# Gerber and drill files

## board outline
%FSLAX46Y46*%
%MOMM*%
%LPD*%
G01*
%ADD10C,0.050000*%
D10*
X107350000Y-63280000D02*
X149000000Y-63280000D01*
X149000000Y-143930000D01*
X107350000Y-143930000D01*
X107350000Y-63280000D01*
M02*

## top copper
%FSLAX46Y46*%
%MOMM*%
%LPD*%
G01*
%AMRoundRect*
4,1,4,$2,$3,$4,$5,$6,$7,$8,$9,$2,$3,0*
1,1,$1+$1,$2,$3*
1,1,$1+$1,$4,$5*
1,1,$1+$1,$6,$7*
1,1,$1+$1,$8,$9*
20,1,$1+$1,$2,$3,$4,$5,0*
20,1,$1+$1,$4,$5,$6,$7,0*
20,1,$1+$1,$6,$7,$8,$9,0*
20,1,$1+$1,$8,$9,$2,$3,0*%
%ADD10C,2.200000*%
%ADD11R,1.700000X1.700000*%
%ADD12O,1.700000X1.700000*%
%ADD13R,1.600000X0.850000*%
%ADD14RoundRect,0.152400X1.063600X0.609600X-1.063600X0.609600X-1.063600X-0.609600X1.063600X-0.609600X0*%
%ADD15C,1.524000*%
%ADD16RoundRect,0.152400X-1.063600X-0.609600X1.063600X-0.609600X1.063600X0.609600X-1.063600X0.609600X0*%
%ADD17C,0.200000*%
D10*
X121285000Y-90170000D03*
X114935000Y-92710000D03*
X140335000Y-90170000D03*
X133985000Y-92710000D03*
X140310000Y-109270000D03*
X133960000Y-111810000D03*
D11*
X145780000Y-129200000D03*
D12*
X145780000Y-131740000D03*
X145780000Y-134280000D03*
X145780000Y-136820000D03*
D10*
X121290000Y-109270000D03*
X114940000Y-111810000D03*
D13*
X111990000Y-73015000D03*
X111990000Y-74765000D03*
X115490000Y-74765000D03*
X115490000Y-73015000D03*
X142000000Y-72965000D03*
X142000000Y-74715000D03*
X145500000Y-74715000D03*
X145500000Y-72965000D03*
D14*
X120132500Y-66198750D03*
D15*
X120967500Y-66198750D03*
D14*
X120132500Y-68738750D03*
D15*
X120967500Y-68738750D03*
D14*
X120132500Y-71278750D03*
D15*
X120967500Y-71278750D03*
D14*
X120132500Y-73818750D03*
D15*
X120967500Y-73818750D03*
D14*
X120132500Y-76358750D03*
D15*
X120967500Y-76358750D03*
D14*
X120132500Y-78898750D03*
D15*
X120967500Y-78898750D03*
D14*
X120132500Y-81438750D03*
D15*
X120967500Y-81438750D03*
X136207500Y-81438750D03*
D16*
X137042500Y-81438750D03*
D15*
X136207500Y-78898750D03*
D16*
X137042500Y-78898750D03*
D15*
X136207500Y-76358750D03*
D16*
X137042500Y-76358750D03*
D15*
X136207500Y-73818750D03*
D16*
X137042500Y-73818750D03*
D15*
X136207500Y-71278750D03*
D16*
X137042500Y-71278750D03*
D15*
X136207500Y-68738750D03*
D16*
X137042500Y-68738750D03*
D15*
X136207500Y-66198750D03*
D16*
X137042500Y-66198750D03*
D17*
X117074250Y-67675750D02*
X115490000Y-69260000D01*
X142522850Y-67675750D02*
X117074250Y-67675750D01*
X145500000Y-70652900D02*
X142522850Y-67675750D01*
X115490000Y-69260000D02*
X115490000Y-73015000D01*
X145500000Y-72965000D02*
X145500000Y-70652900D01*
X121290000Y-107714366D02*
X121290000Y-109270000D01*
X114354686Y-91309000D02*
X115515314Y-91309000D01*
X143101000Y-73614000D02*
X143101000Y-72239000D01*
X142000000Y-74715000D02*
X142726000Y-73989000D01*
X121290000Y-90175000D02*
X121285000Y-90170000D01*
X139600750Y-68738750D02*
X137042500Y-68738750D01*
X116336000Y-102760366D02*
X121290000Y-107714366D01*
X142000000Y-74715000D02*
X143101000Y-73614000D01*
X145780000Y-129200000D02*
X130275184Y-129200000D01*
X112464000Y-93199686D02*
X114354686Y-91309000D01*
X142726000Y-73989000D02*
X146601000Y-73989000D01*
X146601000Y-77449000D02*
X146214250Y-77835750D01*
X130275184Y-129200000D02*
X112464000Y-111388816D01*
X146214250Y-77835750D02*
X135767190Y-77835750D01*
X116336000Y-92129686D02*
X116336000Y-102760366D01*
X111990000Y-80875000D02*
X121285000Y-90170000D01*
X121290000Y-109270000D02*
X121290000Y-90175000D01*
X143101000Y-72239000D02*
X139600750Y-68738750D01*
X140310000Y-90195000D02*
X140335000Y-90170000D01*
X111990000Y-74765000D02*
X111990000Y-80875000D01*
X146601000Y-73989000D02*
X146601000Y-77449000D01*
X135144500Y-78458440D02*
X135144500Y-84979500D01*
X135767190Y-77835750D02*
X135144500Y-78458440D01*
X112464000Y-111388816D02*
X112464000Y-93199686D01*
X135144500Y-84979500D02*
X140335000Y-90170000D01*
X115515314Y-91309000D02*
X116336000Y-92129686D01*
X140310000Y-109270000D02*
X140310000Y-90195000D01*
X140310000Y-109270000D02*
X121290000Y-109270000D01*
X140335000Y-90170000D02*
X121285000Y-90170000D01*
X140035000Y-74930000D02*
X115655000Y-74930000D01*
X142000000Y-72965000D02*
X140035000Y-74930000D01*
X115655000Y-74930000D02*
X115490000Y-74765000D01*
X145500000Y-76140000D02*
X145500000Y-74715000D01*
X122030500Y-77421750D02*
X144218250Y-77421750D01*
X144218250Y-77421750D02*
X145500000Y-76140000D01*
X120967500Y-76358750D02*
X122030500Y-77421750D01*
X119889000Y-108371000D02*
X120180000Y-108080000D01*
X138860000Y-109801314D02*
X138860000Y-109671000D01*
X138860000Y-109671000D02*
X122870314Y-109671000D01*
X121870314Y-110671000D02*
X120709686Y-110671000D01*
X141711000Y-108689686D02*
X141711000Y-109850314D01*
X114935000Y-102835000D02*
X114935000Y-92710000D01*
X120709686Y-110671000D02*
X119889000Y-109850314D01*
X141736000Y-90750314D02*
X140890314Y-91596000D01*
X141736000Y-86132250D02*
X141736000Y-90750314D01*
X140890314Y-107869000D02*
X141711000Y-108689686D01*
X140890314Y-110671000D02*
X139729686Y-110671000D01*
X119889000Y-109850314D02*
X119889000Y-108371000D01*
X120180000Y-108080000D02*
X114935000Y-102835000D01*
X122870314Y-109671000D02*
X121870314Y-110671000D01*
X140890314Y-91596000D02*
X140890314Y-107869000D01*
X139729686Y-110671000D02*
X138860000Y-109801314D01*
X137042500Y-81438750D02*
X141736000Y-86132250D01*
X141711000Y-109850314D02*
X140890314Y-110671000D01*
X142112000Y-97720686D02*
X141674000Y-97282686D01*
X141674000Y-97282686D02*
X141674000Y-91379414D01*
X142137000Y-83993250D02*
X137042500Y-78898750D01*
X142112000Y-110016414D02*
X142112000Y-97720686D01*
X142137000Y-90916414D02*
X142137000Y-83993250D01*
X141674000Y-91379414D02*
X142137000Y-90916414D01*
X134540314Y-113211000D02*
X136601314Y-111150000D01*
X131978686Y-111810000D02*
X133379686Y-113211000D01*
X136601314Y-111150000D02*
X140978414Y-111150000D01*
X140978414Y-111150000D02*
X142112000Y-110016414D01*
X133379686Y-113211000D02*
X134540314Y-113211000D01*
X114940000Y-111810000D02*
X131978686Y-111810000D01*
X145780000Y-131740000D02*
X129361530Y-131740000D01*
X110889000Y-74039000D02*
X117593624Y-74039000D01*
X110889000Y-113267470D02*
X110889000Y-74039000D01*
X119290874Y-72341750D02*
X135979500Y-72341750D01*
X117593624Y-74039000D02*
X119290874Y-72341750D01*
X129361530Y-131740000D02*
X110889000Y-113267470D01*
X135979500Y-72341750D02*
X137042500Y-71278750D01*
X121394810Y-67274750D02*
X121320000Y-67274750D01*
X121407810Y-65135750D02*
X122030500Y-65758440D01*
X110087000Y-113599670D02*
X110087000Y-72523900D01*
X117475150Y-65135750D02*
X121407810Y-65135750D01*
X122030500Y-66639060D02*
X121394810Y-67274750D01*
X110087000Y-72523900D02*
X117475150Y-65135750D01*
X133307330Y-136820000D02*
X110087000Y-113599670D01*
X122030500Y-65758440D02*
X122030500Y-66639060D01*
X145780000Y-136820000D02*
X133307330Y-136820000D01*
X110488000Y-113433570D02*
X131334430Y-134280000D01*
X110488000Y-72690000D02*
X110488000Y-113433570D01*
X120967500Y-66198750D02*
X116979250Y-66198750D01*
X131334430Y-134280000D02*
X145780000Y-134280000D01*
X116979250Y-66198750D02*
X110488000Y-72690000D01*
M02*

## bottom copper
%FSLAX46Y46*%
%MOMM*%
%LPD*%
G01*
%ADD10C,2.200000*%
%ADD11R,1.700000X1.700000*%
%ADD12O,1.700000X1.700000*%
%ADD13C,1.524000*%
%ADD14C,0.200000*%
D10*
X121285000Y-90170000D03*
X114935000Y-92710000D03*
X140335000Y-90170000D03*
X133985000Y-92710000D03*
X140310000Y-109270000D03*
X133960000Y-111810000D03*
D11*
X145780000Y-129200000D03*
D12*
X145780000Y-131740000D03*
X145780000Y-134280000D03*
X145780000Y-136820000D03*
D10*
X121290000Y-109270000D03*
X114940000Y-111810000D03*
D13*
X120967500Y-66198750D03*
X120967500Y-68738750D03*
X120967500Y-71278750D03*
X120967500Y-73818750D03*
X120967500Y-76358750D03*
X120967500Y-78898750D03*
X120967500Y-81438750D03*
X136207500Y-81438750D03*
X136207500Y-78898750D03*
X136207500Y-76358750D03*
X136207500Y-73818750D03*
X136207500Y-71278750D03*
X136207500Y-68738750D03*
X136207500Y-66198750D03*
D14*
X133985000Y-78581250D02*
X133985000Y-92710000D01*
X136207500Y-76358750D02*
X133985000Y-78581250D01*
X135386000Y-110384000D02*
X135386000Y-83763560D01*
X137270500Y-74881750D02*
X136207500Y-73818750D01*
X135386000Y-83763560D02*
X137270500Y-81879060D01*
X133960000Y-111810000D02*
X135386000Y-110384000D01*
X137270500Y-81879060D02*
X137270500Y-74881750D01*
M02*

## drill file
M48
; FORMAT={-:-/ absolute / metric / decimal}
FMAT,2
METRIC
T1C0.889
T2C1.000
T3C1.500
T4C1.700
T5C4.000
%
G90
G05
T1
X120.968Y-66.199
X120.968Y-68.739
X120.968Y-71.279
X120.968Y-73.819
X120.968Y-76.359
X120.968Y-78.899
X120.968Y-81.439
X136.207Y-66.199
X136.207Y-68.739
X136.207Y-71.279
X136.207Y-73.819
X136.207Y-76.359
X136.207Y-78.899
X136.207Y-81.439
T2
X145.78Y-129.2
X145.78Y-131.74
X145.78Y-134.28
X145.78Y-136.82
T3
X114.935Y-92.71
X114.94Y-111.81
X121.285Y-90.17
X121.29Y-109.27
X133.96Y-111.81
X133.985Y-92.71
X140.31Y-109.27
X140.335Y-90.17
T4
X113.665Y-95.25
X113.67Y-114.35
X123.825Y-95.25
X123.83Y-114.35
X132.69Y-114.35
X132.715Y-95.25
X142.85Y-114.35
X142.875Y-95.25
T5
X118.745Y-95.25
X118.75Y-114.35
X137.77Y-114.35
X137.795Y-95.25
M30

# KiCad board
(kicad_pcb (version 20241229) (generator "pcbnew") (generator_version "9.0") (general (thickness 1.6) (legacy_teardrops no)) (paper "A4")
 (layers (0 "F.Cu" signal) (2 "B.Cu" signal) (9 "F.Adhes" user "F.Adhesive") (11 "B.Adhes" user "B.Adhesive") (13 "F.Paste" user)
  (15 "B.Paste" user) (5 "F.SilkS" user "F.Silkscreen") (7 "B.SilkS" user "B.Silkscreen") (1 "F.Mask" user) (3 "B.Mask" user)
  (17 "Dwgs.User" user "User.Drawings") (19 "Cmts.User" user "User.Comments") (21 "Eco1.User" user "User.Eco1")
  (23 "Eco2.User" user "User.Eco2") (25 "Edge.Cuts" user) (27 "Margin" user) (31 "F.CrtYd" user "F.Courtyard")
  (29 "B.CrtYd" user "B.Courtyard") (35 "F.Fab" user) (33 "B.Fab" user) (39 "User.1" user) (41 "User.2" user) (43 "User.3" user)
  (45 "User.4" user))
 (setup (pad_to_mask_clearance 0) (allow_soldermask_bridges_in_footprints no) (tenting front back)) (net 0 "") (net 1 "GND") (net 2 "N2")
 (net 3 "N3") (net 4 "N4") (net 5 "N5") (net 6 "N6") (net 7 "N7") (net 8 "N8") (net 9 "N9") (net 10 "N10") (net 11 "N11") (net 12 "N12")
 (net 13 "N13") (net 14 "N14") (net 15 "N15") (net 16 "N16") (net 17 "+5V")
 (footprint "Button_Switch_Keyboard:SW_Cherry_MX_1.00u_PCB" (layer "F.Cu") (at 121.285 90.17)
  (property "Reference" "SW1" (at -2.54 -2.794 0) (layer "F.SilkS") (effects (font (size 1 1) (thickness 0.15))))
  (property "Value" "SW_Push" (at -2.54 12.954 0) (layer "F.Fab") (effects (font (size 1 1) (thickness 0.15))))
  (pad "" np_thru_hole circle (at -7.62 5.08) (size 1.7 1.7) (drill 1.7) (layers "*.Cu" "*.Mask"))
  (pad "" np_thru_hole circle (at -2.54 5.08) (size 4 4) (drill 4) (layers "*.Cu" "*.Mask"))
  (pad "" np_thru_hole circle (at 2.54 5.08) (size 1.7 1.7) (drill 1.7) (layers "*.Cu" "*.Mask"))
  (pad "1" thru_hole circle (at 0 0) (size 2.2 2.2) (drill 1.5) (layers "*.Cu" "*.Mask") (remove_unused_layers no) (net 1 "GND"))
  (pad "2" thru_hole circle (at -6.35 2.54) (size 2.2 2.2) (drill 1.5) (layers "*.Cu" "*.Mask") (remove_unused_layers no) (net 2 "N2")))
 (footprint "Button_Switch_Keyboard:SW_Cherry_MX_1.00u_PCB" (layer "F.Cu") (at 140.335 90.17)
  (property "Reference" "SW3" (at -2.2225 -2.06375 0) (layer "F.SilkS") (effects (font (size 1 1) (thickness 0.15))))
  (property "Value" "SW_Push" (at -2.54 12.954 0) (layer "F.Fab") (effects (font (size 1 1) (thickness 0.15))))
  (pad "" np_thru_hole circle (at -7.62 5.08) (size 1.7 1.7) (drill 1.7) (layers "*.Cu" "*.Mask"))
  (pad "" np_thru_hole circle (at -2.54 5.08) (size 4 4) (drill 4) (layers "*.Cu" "*.Mask"))
  (pad "" np_thru_hole circle (at 2.54 5.08) (size 1.7 1.7) (drill 1.7) (layers "*.Cu" "*.Mask"))
  (pad "1" thru_hole circle (at 0 0) (size 2.2 2.2) (drill 1.5) (layers "*.Cu" "*.Mask") (remove_unused_layers no) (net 1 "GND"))
  (pad "2" thru_hole circle (at -6.35 2.54) (size 2.2 2.2) (drill 1.5) (layers "*.Cu" "*.Mask") (remove_unused_layers no) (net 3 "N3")))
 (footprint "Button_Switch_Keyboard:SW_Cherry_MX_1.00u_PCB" (layer "F.Cu") (at 140.31 109.27)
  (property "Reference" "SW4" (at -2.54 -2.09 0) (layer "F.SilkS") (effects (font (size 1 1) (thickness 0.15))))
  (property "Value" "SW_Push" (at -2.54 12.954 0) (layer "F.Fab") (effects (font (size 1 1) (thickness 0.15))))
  (pad "" np_thru_hole circle (at -7.62 5.08) (size 1.7 1.7) (drill 1.7) (layers "*.Cu" "*.Mask"))
  (pad "" np_thru_hole circle (at -2.54 5.08) (size 4 4) (drill 4) (layers "*.Cu" "*.Mask"))
  (pad "" np_thru_hole circle (at 2.54 5.08) (size 1.7 1.7) (drill 1.7) (layers "*.Cu" "*.Mask"))
  (pad "1" thru_hole circle (at 0 0) (size 2.2 2.2) (drill 1.5) (layers "*.Cu" "*.Mask") (remove_unused_layers no) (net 1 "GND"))
  (pad "2" thru_hole circle (at -6.35 2.54) (size 2.2 2.2) (drill 1.5) (layers "*.Cu" "*.Mask") (remove_unused_layers no) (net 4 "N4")))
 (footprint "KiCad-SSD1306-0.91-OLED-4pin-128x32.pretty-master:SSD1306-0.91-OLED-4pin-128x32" (layer "F.Cu") (at 109.28 127.01)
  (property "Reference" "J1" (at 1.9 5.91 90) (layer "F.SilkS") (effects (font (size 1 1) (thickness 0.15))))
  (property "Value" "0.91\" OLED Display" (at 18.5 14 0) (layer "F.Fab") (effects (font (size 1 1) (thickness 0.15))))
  (pad "1" thru_hole rect (at 36.5 2.19) (size 1.7 1.7) (drill 1) (layers "*.Cu" "*.Mask") (remove_unused_layers no) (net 1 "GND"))
  (pad "2" thru_hole oval (at 36.5 4.73) (size 1.7 1.7) (drill 1) (layers "*.Cu" "*.Mask") (remove_unused_layers no) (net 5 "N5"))
  (pad "3" thru_hole oval (at 36.5 7.27) (size 1.7 1.7) (drill 1) (layers "*.Cu" "*.Mask") (remove_unused_layers no) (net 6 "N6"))
  (pad "4" thru_hole oval (at 36.5 9.81) (size 1.7 1.7) (drill 1) (layers "*.Cu" "*.Mask") (remove_unused_layers no) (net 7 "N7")))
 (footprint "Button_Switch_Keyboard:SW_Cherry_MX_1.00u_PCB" (layer "F.Cu") (at 121.29 109.27)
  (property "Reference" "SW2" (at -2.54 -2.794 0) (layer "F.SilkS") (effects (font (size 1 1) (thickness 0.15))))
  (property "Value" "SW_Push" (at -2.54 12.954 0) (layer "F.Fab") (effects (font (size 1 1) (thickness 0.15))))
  (pad "" np_thru_hole circle (at -7.62 5.08) (size 1.7 1.7) (drill 1.7) (layers "*.Cu" "*.Mask"))
  (pad "" np_thru_hole circle (at -2.54 5.08) (size 4 4) (drill 4) (layers "*.Cu" "*.Mask"))
  (pad "" np_thru_hole circle (at 2.54 5.08) (size 1.7 1.7) (drill 1.7) (layers "*.Cu" "*.Mask"))
  (pad "1" thru_hole circle (at 0 0) (size 2.2 2.2) (drill 1.5) (layers "*.Cu" "*.Mask") (remove_unused_layers no) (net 1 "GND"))
  (pad "2" thru_hole circle (at -6.35 2.54) (size 2.2 2.2) (drill 1.5) (layers "*.Cu" "*.Mask") (remove_unused_layers no) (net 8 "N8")))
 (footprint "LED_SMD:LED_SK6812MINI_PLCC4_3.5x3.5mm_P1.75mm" (layer "F.Cu") (at 113.74 73.89)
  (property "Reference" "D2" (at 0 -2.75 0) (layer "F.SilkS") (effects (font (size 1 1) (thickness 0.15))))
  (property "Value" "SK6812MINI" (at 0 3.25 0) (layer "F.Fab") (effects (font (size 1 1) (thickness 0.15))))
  (pad "1" smd rect (at -1.75 -0.875) (size 1.6 0.85) (layers "F.Cu" "F.Mask" "F.Paste") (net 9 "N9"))
  (pad "2" smd rect (at -1.75 0.875) (size 1.6 0.85) (layers "F.Cu" "F.Mask" "F.Paste") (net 1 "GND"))
  (pad "3" smd rect (at 1.75 0.875) (size 1.6 0.85) (layers "F.Cu" "F.Mask" "F.Paste") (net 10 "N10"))
  (pad "4" smd rect (at 1.75 -0.875) (size 1.6 0.85) (layers "F.Cu" "F.Mask" "F.Paste") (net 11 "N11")))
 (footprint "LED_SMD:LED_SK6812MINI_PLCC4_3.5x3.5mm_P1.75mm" (layer "F.Cu") (at 143.75 73.84)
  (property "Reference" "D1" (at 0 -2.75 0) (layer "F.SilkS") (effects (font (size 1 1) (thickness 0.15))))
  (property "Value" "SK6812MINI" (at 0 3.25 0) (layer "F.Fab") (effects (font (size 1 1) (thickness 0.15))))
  (pad "1" smd rect (at -1.75 -0.875) (size 1.6 0.85) (layers "F.Cu" "F.Mask" "F.Paste") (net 10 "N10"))
  (pad "2" smd rect (at -1.75 0.875) (size 1.6 0.85) (layers "F.Cu" "F.Mask" "F.Paste") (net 1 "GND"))
  (pad "3" smd rect (at 1.75 0.875) (size 1.6 0.85) (layers "F.Cu" "F.Mask" "F.Paste") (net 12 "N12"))
  (pad "4" smd rect (at 1.75 -0.875) (size 1.6 0.85) (layers "F.Cu" "F.Mask" "F.Paste") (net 11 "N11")))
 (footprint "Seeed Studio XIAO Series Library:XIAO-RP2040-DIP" (layer "F.Cu") (at 128.5875 73.81875)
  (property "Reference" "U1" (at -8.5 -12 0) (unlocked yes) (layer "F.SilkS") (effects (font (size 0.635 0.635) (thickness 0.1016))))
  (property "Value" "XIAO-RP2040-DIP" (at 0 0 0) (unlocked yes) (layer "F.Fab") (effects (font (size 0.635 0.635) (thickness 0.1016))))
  (pad "1" smd roundrect (at -8.455 -7.62 180) (size 2.432 1.524) (layers "F.Cu" "F.Mask") (roundrect_rratio 0.1) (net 6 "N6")
   (thermal_bridge_angle 45))
  (pad "1" thru_hole circle (at -7.62 -7.62 180) (size 1.524 1.524) (drill 0.889) (layers "*.Cu" "*.Mask") (remove_unused_layers no)
   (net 6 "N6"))
  (pad "2" smd roundrect (at -8.455 -5.08 180) (size 2.432 1.524) (layers "F.Cu" "F.Mask") (roundrect_rratio 0.1) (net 7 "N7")
   (thermal_bridge_angle 45))
  (pad "2" thru_hole circle (at -7.62 -5.08 180) (size 1.524 1.524) (drill 0.889) (layers "*.Cu" "*.Mask") (remove_unused_layers no)
   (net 7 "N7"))
  (pad "3" smd roundrect (at -8.455 -2.54 180) (size 2.432 1.524) (layers "F.Cu" "F.Mask") (roundrect_rratio 0.1) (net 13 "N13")
   (thermal_bridge_angle 45))
  (pad "3" thru_hole circle (at -7.62 -2.54 180) (size 1.524 1.524) (drill 0.889) (layers "*.Cu" "*.Mask") (remove_unused_layers no)
   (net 13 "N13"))
  (pad "4" smd roundrect (at -8.455 0 180) (size 2.432 1.524) (layers "F.Cu" "F.Mask") (roundrect_rratio 0.1) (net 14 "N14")
   (thermal_bridge_angle 45))
  (pad "4" thru_hole circle (at -7.62 0 180) (size 1.524 1.524) (drill 0.889) (layers "*.Cu" "*.Mask") (remove_unused_layers no)
   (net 14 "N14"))
  (pad "5" smd roundrect (at -8.455 2.54 180) (size 2.432 1.524) (layers "F.Cu" "F.Mask") (roundrect_rratio 0.1) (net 12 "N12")
   (thermal_bridge_angle 45))
  (pad "5" thru_hole circle (at -7.62 2.54 180) (size 1.524 1.524) (drill 0.889) (layers "*.Cu" "*.Mask") (remove_unused_layers no)
   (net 12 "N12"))
  (pad "6" smd roundrect (at -8.455 5.08 180) (size 2.432 1.524) (layers "F.Cu" "F.Mask") (roundrect_rratio 0.1) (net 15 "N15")
   (thermal_bridge_angle 45))
  (pad "6" thru_hole circle (at -7.62 5.08 180) (size 1.524 1.524) (drill 0.889) (layers "*.Cu" "*.Mask") (remove_unused_layers no)
   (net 15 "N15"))
  (pad "7" smd roundrect (at -8.455 7.62 180) (size 2.432 1.524) (layers "F.Cu" "F.Mask") (roundrect_rratio 0.1) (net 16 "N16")
   (thermal_bridge_angle 45))
  (pad "7" thru_hole circle (at -7.62 7.62 180) (size 1.524 1.524) (drill 0.889) (layers "*.Cu" "*.Mask") (remove_unused_layers no)
   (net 16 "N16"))
  (pad "8" thru_hole circle (at 7.62 7.62) (size 1.524 1.524) (drill 0.889) (layers "*.Cu" "*.Mask") (remove_unused_layers no) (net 2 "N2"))
  (pad "8" smd roundrect (at 8.455 7.62) (size 2.432 1.524) (layers "F.Cu" "F.Mask") (roundrect_rratio 0.1) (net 2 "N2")
   (thermal_bridge_angle 45))
  (pad "9" thru_hole circle (at 7.62 5.08) (size 1.524 1.524) (drill 0.889) (layers "*.Cu" "*.Mask") (remove_unused_layers no) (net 8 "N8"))
  (pad "9" smd roundrect (at 8.455 5.08) (size 2.432 1.524) (layers "F.Cu" "F.Mask") (roundrect_rratio 0.1) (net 8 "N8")
   (thermal_bridge_angle 45))
  (pad "10" thru_hole circle (at 7.62 2.54) (size 1.524 1.524) (drill 0.889) (layers "*.Cu" "*.Mask") (remove_unused_layers no) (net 3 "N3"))
  (pad "10" smd roundrect (at 8.455 2.54) (size 2.432 1.524) (layers "F.Cu" "F.Mask") (roundrect_rratio 0.1) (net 3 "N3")
   (thermal_bridge_angle 45))
  (pad "11" thru_hole circle (at 7.62 0) (size 1.524 1.524) (drill 0.889) (layers "*.Cu" "*.Mask") (remove_unused_layers no) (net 4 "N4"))
  (pad "11" smd roundrect (at 8.455 0) (size 2.432 1.524) (layers "F.Cu" "F.Mask") (roundrect_rratio 0.1) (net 4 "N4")
   (thermal_bridge_angle 45))
  (pad "12" thru_hole circle (at 7.62 -2.54) (size 1.524 1.524) (drill 0.889) (layers "*.Cu" "*.Mask") (remove_unused_layers no)
   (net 5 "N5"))
  (pad "12" smd roundrect (at 8.455 -2.54) (size 2.432 1.524) (layers "F.Cu" "F.Mask") (roundrect_rratio 0.1) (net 5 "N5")
   (thermal_bridge_angle 45))
  (pad "13" thru_hole circle (at 7.62 -5.08) (size 1.524 1.524) (drill 0.889) (layers "*.Cu" "*.Mask") (remove_unused_layers no)
   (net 1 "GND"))
  (pad "13" smd roundrect (at 8.455 -5.08) (size 2.432 1.524) (layers "F.Cu" "F.Mask") (roundrect_rratio 0.1) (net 1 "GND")
   (thermal_bridge_angle 45))
  (pad "14" thru_hole circle (at 7.62 -7.62) (size 1.524 1.524) (drill 0.889) (layers "*.Cu" "*.Mask") (remove_unused_layers no)
   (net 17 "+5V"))
  (pad "14" smd roundrect (at 8.455 -7.62) (size 2.432 1.524) (layers "F.Cu" "F.Mask") (roundrect_rratio 0.1) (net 17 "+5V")
   (thermal_bridge_angle 45)))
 (gr_rect (start 107.35 63.28) (end 149 143.93) (stroke (width 0.05) (type default)) (fill no) (layer "Edge.Cuts"))
 (segment (start 117.07425 67.67575) (end 115.49 69.26) (width 0.2) (layer "F.Cu") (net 11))
 (segment (start 142.52285 67.67575) (end 117.07425 67.67575) (width 0.2) (layer "F.Cu") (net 11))
 (segment (start 145.5 70.6529) (end 142.52285 67.67575) (width 0.2) (layer "F.Cu") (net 11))
 (segment (start 115.49 69.26) (end 115.49 73.015) (width 0.2) (layer "F.Cu") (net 11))
 (segment (start 145.5 72.965) (end 145.5 70.6529) (width 0.2) (layer "F.Cu") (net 11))
 (segment (start 121.29 107.714366) (end 121.29 109.27) (width 0.2) (layer "F.Cu") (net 1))
 (segment (start 114.354686 91.309) (end 115.515314 91.309) (width 0.2) (layer "F.Cu") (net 1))
 (segment (start 143.101 73.614) (end 143.101 72.239) (width 0.2) (layer "F.Cu") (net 1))
 (segment (start 142 74.715) (end 142.726 73.989) (width 0.2) (layer "F.Cu") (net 1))
 (segment (start 121.29 90.175) (end 121.285 90.17) (width 0.2) (layer "F.Cu") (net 1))
 (segment (start 139.60075 68.73875) (end 137.0425 68.73875) (width 0.2) (layer "F.Cu") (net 1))
 (segment (start 116.336 102.760366) (end 121.29 107.714366) (width 0.2) (layer "F.Cu") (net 1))
 (segment (start 142 74.715) (end 143.101 73.614) (width 0.2) (layer "F.Cu") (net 1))
 (segment (start 145.78 129.2) (end 130.275184 129.2) (width 0.2) (layer "F.Cu") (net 1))
 (segment (start 112.464 93.199686) (end 114.354686 91.309) (width 0.2) (layer "F.Cu") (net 1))
 (segment (start 142.726 73.989) (end 146.601 73.989) (width 0.2) (layer "F.Cu") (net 1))
 (segment (start 146.601 77.449) (end 146.21425 77.83575) (width 0.2) (layer "F.Cu") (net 1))
 (segment (start 130.275184 129.2) (end 112.464 111.388816) (width 0.2) (layer "F.Cu") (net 1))
 (segment (start 146.21425 77.83575) (end 135.76719 77.83575) (width 0.2) (layer "F.Cu") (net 1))
 (segment (start 116.336 92.129686) (end 116.336 102.760366) (width 0.2) (layer "F.Cu") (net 1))
 (segment (start 111.99 80.875) (end 121.285 90.17) (width 0.2) (layer "F.Cu") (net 1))
 (segment (start 121.29 109.27) (end 121.29 90.175) (width 0.2) (layer "F.Cu") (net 1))
 (segment (start 143.101 72.239) (end 139.60075 68.73875) (width 0.2) (layer "F.Cu") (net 1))
 (segment (start 140.31 90.195) (end 140.335 90.17) (width 0.2) (layer "F.Cu") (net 1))
 (segment (start 111.99 74.765) (end 111.99 80.875) (width 0.2) (layer "F.Cu") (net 1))
 (segment (start 146.601 73.989) (end 146.601 77.449) (width 0.2) (layer "F.Cu") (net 1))
 (segment (start 135.1445 78.45844) (end 135.1445 84.9795) (width 0.2) (layer "F.Cu") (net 1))
 (segment (start 135.76719 77.83575) (end 135.1445 78.45844) (width 0.2) (layer "F.Cu") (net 1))
 (segment (start 112.464 111.388816) (end 112.464 93.199686) (width 0.2) (layer "F.Cu") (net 1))
 (segment (start 135.1445 84.9795) (end 140.335 90.17) (width 0.2) (layer "F.Cu") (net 1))
 (segment (start 115.515314 91.309) (end 116.336 92.129686) (width 0.2) (layer "F.Cu") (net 1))
 (segment (start 140.31 109.27) (end 140.31 90.195) (width 0.2) (layer "F.Cu") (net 1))
 (segment (start 140.31 109.27) (end 121.29 109.27) (width 0.2) (layer "F.Cu") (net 1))
 (segment (start 140.335 90.17) (end 121.285 90.17) (width 0.2) (layer "F.Cu") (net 1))
 (segment (start 140.035 74.93) (end 115.655 74.93) (width 0.2) (layer "F.Cu") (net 10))
 (segment (start 142 72.965) (end 140.035 74.93) (width 0.2) (layer "F.Cu") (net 10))
 (segment (start 115.655 74.93) (end 115.49 74.765) (width 0.2) (layer "F.Cu") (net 10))
 (segment (start 145.5 76.14) (end 145.5 74.715) (width 0.2) (layer "F.Cu") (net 12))
 (segment (start 122.0305 77.42175) (end 144.21825 77.42175) (width 0.2) (layer "F.Cu") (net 12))
 (segment (start 144.21825 77.42175) (end 145.5 76.14) (width 0.2) (layer "F.Cu") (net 12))
 (segment (start 120.9675 76.35875) (end 122.0305 77.42175) (width 0.2) (layer "F.Cu") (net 12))
 (segment (start 119.889 108.371) (end 120.18 108.08) (width 0.2) (layer "F.Cu") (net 2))
 (segment (start 138.86 109.801314) (end 138.86 109.671) (width 0.2) (layer "F.Cu") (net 2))
 (segment (start 138.86 109.671) (end 122.870314 109.671) (width 0.2) (layer "F.Cu") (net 2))
 (segment (start 121.870314 110.671) (end 120.709686 110.671) (width 0.2) (layer "F.Cu") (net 2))
 (segment (start 141.711 108.689686) (end 141.711 109.850314) (width 0.2) (layer "F.Cu") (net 2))
 (segment (start 114.935 102.835) (end 114.935 92.71) (width 0.2) (layer "F.Cu") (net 2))
 (segment (start 120.709686 110.671) (end 119.889 109.850314) (width 0.2) (layer "F.Cu") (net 2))
 (segment (start 141.736 90.750314) (end 140.890314 91.596) (width 0.2) (layer "F.Cu") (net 2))
 (segment (start 141.736 86.13225) (end 141.736 90.750314) (width 0.2) (layer "F.Cu") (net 2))
 (segment (start 140.890314 107.869) (end 141.711 108.689686) (width 0.2) (layer "F.Cu") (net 2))
 (segment (start 140.890314 110.671) (end 139.729686 110.671) (width 0.2) (layer "F.Cu") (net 2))
 (segment (start 119.889 109.850314) (end 119.889 108.371) (width 0.2) (layer "F.Cu") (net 2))
 (segment (start 120.18 108.08) (end 114.935 102.835) (width 0.2) (layer "F.Cu") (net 2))
 (segment (start 122.870314 109.671) (end 121.870314 110.671) (width 0.2) (layer "F.Cu") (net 2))
 (segment (start 140.890314 91.596) (end 140.890314 107.869) (width 0.2) (layer "F.Cu") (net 2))
 (segment (start 139.729686 110.671) (end 138.86 109.801314) (width 0.2) (layer "F.Cu") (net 2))
 (segment (start 137.0425 81.43875) (end 141.736 86.13225) (width 0.2) (layer "F.Cu") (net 2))
 (segment (start 141.711 109.850314) (end 140.890314 110.671) (width 0.2) (layer "F.Cu") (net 2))
 (segment (start 142.112 97.720686) (end 141.674 97.282686) (width 0.2) (layer "F.Cu") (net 8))
 (segment (start 141.674 97.282686) (end 141.674 91.379414) (width 0.2) (layer "F.Cu") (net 8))
 (segment (start 142.137 83.99325) (end 137.0425 78.89875) (width 0.2) (layer "F.Cu") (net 8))
 (segment (start 142.112 110.016414) (end 142.112 97.720686) (width 0.2) (layer "F.Cu") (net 8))
 (segment (start 142.137 90.916414) (end 142.137 83.99325) (width 0.2) (layer "F.Cu") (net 8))
 (segment (start 141.674 91.379414) (end 142.137 90.916414) (width 0.2) (layer "F.Cu") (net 8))
 (segment (start 134.540314 113.211) (end 136.601314 111.15) (width 0.2) (layer "F.Cu") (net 8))
 (segment (start 131.978686 111.81) (end 133.379686 113.211) (width 0.2) (layer "F.Cu") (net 8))
 (segment (start 136.601314 111.15) (end 140.978414 111.15) (width 0.2) (layer "F.Cu") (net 8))
 (segment (start 140.978414 111.15) (end 142.112 110.016414) (width 0.2) (layer "F.Cu") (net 8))
 (segment (start 133.379686 113.211) (end 134.540314 113.211) (width 0.2) (layer "F.Cu") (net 8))
 (segment (start 114.94 111.81) (end 131.978686 111.81) (width 0.2) (layer "F.Cu") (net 8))
 (segment (start 133.985 78.58125) (end 133.985 92.71) (width 0.2) (layer "B.Cu") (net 3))
 (segment (start 136.2075 76.35875) (end 133.985 78.58125) (width 0.2) (layer "B.Cu") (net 3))
 (segment (start 135.386 110.384) (end 135.386 83.76356) (width 0.2) (layer "B.Cu") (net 4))
 (segment (start 137.2705 74.88175) (end 136.2075 73.81875) (width 0.2) (layer "B.Cu") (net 4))
 (segment (start 135.386 83.76356) (end 137.2705 81.87906) (width 0.2) (layer "B.Cu") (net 4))
 (segment (start 133.96 111.81) (end 135.386 110.384) (width 0.2) (layer "B.Cu") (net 4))
 (segment (start 137.2705 81.87906) (end 137.2705 74.88175) (width 0.2) (layer "B.Cu") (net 4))
 (segment (start 145.78 131.74) (end 129.36153 131.74) (width 0.2) (layer "F.Cu") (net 5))
 (segment (start 110.889 74.039) (end 117.593624 74.039) (width 0.2) (layer "F.Cu") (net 5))
 (segment (start 110.889 113.26747) (end 110.889 74.039) (width 0.2) (layer "F.Cu") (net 5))
 (segment (start 119.290874 72.34175) (end 135.9795 72.34175) (width 0.2) (layer "F.Cu") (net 5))
 (segment (start 117.593624 74.039) (end 119.290874 72.34175) (width 0.2) (layer "F.Cu") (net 5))
 (segment (start 129.36153 131.74) (end 110.889 113.26747) (width 0.2) (layer "F.Cu") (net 5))
 (segment (start 135.9795 72.34175) (end 137.0425 71.27875) (width 0.2) (layer "F.Cu") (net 5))
 (segment (start 121.39481 67.27475) (end 121.32 67.27475) (width 0.2) (layer "F.Cu") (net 7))
 (segment (start 121.40781 65.13575) (end 122.0305 65.75844) (width 0.2) (layer "F.Cu") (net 7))
 (segment (start 110.087 113.59967) (end 110.087 72.5239) (width 0.2) (layer "F.Cu") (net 7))
 (segment (start 117.47515 65.13575) (end 121.40781 65.13575) (width 0.2) (layer "F.Cu") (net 7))
 (segment (start 122.0305 66.63906) (end 121.39481 67.27475) (width 0.2) (layer "F.Cu") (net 7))
 (segment (start 110.087 72.5239) (end 117.47515 65.13575) (width 0.2) (layer "F.Cu") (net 7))
 (segment (start 133.30733 136.82) (end 110.087 113.59967) (width 0.2) (layer "F.Cu") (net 7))
 (segment (start 122.0305 65.75844) (end 122.0305 66.63906) (width 0.2) (layer "F.Cu") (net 7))
 (segment (start 145.78 136.82) (end 133.30733 136.82) (width 0.2) (layer "F.Cu") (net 7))
 (segment (start 110.488 113.43357) (end 131.33443 134.28) (width 0.2) (layer "F.Cu") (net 6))
 (segment (start 110.488 72.69) (end 110.488 113.43357) (width 0.2) (layer "F.Cu") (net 6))
 (segment (start 120.9675 66.19875) (end 116.97925 66.19875) (width 0.2) (layer "F.Cu") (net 6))
 (segment (start 131.33443 134.28) (end 145.78 134.28) (width 0.2) (layer "F.Cu") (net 6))
 (segment (start 116.97925 66.19875) (end 110.488 72.69) (width 0.2) (layer "F.Cu") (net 6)))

